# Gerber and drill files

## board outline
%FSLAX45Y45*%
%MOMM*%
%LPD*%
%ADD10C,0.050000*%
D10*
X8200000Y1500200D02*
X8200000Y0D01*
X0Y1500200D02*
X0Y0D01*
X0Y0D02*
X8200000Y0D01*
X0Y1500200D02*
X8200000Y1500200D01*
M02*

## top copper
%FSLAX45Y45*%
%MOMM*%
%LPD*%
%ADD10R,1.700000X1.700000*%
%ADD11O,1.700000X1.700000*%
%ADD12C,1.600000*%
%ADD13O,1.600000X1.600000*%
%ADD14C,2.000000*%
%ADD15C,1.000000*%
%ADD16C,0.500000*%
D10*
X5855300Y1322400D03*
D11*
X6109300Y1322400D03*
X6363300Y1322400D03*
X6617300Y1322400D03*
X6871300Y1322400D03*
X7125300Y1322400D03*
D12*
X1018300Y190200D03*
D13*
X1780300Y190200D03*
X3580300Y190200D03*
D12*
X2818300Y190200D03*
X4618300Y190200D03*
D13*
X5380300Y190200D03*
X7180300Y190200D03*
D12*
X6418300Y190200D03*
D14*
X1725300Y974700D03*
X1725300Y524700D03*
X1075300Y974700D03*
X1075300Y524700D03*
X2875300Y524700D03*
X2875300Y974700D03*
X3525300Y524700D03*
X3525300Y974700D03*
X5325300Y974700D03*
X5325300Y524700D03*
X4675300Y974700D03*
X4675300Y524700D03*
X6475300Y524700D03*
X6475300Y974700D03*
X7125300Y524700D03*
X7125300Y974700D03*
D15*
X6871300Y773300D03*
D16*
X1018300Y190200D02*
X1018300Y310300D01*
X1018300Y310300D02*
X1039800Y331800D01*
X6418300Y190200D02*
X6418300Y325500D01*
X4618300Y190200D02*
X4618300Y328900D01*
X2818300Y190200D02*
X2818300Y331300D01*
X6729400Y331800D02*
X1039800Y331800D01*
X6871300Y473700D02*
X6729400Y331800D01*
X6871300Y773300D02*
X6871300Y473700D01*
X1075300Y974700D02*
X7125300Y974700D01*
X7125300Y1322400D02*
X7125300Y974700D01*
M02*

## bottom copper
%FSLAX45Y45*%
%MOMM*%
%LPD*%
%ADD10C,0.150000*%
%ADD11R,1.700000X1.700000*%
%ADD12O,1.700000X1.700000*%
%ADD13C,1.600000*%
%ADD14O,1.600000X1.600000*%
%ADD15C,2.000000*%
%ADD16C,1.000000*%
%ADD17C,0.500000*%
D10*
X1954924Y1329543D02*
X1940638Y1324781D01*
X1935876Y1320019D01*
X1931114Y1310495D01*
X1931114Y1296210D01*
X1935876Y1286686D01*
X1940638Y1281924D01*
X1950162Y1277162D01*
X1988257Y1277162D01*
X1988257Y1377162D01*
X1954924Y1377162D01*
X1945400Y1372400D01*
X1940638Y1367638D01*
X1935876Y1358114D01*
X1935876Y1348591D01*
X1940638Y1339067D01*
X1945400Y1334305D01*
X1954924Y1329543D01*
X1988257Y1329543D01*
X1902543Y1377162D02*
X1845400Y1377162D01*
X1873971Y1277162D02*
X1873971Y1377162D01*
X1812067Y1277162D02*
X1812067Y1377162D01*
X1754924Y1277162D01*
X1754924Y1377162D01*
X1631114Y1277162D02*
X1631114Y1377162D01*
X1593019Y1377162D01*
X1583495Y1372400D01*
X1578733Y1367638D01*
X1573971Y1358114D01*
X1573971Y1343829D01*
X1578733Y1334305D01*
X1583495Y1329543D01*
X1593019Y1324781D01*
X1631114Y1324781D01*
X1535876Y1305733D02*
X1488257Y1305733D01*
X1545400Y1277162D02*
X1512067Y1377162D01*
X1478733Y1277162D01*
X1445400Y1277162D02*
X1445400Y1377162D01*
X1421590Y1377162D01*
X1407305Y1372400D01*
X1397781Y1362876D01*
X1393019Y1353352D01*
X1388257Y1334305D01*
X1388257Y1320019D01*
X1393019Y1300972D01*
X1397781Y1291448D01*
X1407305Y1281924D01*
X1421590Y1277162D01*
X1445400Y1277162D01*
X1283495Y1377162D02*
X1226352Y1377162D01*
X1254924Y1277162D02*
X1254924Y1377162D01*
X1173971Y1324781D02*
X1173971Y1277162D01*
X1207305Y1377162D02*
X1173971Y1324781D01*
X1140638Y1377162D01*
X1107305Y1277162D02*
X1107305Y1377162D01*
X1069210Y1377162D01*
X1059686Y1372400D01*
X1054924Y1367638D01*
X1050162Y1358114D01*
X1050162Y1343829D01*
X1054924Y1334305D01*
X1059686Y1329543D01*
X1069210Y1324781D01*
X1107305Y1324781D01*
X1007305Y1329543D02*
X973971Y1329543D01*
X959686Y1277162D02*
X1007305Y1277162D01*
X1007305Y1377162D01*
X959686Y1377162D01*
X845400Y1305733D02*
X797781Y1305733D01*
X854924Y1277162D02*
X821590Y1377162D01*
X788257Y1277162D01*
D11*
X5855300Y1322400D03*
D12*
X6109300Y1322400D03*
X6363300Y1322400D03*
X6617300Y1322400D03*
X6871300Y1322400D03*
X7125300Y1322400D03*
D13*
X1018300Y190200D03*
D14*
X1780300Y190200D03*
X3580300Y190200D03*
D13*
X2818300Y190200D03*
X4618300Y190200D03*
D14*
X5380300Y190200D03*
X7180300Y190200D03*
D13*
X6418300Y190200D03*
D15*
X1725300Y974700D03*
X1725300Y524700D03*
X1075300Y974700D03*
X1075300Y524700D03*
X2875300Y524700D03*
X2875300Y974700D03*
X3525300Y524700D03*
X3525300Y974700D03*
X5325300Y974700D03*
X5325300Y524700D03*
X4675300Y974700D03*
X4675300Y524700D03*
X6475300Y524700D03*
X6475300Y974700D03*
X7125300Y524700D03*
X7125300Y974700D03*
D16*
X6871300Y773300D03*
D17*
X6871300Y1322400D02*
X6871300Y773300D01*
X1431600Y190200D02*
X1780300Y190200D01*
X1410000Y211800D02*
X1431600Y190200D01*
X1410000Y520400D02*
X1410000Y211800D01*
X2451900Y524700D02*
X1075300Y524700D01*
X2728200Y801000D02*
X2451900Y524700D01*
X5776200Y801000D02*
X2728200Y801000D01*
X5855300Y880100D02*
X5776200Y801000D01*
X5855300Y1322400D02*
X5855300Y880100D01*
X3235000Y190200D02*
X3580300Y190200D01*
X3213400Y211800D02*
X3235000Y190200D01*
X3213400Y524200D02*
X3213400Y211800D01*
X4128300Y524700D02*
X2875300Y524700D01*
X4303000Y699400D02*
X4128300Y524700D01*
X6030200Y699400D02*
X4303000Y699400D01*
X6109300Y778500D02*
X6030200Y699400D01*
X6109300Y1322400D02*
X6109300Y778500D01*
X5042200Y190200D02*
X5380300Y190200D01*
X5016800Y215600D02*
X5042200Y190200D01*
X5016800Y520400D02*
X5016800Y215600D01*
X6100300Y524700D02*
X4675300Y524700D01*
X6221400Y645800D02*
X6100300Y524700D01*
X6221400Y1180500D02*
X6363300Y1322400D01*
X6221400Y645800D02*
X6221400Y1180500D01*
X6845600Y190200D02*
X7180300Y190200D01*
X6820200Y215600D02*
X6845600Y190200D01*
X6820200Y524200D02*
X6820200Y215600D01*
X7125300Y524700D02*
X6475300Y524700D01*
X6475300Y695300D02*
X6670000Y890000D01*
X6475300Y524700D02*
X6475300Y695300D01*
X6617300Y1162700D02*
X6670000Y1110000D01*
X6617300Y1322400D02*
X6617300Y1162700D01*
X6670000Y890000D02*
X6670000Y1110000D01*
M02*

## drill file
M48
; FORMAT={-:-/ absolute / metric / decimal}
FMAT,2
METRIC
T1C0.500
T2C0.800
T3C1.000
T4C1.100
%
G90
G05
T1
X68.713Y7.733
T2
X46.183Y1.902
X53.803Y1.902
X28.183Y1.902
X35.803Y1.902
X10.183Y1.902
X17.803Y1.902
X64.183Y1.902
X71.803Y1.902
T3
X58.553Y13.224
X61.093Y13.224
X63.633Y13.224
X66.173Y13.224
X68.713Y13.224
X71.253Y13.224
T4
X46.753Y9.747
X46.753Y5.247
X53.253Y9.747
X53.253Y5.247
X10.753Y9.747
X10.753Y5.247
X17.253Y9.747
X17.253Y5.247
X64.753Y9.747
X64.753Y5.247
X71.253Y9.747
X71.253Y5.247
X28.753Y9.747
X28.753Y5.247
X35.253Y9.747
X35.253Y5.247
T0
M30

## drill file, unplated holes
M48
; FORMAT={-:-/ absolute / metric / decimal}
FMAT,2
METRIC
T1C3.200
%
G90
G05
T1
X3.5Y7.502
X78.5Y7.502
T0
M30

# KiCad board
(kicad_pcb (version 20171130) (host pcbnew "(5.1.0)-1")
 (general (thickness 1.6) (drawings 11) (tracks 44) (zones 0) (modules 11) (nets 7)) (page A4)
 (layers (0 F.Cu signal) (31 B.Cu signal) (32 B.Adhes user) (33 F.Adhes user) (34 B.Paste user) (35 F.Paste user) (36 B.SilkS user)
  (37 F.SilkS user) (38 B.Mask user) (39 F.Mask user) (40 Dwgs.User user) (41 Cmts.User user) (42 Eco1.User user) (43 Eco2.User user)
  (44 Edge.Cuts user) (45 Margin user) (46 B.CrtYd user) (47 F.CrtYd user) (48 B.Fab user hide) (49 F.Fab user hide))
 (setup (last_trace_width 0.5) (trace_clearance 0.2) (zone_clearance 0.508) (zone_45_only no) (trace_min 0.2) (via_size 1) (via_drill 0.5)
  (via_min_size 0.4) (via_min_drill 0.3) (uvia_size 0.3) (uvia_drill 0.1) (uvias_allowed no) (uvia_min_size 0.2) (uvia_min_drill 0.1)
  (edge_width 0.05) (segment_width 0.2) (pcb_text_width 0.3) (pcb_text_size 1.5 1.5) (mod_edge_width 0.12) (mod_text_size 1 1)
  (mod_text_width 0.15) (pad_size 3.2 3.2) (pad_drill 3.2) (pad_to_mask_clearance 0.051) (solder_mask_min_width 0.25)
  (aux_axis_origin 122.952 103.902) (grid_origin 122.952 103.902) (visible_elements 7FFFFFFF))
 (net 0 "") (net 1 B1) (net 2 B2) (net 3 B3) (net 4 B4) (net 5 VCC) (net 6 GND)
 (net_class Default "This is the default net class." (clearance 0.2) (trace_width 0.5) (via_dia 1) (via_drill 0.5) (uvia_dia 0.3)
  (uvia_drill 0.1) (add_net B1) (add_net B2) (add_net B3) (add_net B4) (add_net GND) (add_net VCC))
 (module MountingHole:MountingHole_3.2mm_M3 (layer F.Cu) (at 201.452 96.4)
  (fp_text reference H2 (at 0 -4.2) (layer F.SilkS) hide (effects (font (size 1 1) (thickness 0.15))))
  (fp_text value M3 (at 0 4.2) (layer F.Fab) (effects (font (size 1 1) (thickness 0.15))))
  (pad 1 np_thru_hole circle (at 0 0) (size 3.2 3.2) (drill 3.2) (layers *.Cu *.Mask)))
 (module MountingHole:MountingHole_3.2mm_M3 (layer F.Cu) (at 126.452 96.4)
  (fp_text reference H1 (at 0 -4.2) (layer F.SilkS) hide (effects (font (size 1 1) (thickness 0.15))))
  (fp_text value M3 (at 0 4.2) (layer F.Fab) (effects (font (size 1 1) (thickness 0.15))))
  (pad "" np_thru_hole circle (at 0 0) (size 3.2 3.2) (drill 3.2) (layers *.Cu *.Mask)))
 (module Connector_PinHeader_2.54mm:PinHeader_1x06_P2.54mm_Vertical (layer F.Cu) (at 181.505 90.678 90)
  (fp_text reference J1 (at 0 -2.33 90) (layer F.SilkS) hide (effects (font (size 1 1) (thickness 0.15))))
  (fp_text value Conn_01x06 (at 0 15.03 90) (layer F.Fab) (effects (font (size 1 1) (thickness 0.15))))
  (pad 1 thru_hole rect (at 0 0 90) (size 1.7 1.7) (drill 1) (layers *.Cu *.Mask) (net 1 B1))
  (pad 2 thru_hole oval (at 0 2.54 90) (size 1.7 1.7) (drill 1) (layers *.Cu *.Mask) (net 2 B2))
  (pad 3 thru_hole oval (at 0 5.08 90) (size 1.7 1.7) (drill 1) (layers *.Cu *.Mask) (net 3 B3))
  (pad 4 thru_hole oval (at 0 7.62 90) (size 1.7 1.7) (drill 1) (layers *.Cu *.Mask) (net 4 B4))
  (pad 5 thru_hole oval (at 0 10.16 90) (size 1.7 1.7) (drill 1) (layers *.Cu *.Mask) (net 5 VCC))
  (pad 6 thru_hole oval (at 0 12.7 90) (size 1.7 1.7) (drill 1) (layers *.Cu *.Mask) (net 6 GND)))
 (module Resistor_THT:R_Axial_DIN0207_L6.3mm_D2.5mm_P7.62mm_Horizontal (layer F.Cu) (at 133.135 102)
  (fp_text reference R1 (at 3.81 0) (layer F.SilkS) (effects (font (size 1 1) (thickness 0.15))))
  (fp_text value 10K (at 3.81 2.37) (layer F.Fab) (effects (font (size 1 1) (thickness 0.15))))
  (pad 1 thru_hole circle (at 0 0) (size 1.6 1.6) (drill 0.8) (layers *.Cu *.Mask) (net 5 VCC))
  (pad 2 thru_hole oval (at 7.62 0) (size 1.6 1.6) (drill 0.8) (layers *.Cu *.Mask) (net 1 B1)))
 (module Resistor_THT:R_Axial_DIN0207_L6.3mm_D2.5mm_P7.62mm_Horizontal (layer F.Cu) (at 151.135 102)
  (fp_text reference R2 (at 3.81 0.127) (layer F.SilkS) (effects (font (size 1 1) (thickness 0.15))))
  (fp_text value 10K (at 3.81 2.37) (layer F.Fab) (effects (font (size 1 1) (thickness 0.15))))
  (pad 2 thru_hole oval (at 7.62 0) (size 1.6 1.6) (drill 0.8) (layers *.Cu *.Mask) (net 2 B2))
  (pad 1 thru_hole circle (at 0 0) (size 1.6 1.6) (drill 0.8) (layers *.Cu *.Mask) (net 5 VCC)))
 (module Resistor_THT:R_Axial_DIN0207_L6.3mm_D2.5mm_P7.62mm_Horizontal (layer F.Cu) (at 169.135 102)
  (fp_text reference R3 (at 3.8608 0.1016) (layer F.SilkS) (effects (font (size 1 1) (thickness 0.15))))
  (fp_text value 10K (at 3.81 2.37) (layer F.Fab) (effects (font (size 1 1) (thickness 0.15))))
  (pad 1 thru_hole circle (at 0 0) (size 1.6 1.6) (drill 0.8) (layers *.Cu *.Mask) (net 5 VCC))
  (pad 2 thru_hole oval (at 7.62 0) (size 1.6 1.6) (drill 0.8) (layers *.Cu *.Mask) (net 3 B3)))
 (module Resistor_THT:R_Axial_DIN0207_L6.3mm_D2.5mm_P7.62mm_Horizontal (layer F.Cu) (at 187.135 102)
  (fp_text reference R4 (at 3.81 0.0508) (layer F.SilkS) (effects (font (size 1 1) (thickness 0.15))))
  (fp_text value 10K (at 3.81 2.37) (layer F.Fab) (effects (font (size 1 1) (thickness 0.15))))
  (pad 2 thru_hole oval (at 7.62 0) (size 1.6 1.6) (drill 0.8) (layers *.Cu *.Mask) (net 4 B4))
  (pad 1 thru_hole circle (at 0 0) (size 1.6 1.6) (drill 0.8) (layers *.Cu *.Mask) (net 5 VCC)))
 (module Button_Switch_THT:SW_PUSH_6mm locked (layer F.Cu) (at 133.705 94.155)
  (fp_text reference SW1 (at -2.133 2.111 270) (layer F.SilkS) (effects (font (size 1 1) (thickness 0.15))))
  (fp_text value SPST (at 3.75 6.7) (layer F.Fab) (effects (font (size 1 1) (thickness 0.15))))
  (pad 1 thru_hole circle (at 6.5 0 90) (size 2 2) (drill 1.1) (layers *.Cu *.Mask) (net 6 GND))
  (pad 2 thru_hole circle (at 6.5 4.5 90) (size 2 2) (drill 1.1) (layers *.Cu *.Mask) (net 1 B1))
  (pad 1 thru_hole circle (at 0 0 90) (size 2 2) (drill 1.1) (layers *.Cu *.Mask) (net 6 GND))
  (pad 2 thru_hole circle (at 0 4.5 90) (size 2 2) (drill 1.1) (layers *.Cu *.Mask) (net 1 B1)))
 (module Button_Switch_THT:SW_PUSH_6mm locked (layer F.Cu) (at 151.705 94.155)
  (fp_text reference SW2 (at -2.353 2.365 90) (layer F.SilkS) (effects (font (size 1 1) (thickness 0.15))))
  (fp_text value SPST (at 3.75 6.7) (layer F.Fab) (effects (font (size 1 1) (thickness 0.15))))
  (pad 2 thru_hole circle (at 0 4.5 90) (size 2 2) (drill 1.1) (layers *.Cu *.Mask) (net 2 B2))
  (pad 1 thru_hole circle (at 0 0 90) (size 2 2) (drill 1.1) (layers *.Cu *.Mask) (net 6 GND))
  (pad 2 thru_hole circle (at 6.5 4.5 90) (size 2 2) (drill 1.1) (layers *.Cu *.Mask) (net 2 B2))
  (pad 1 thru_hole circle (at 6.5 0 90) (size 2 2) (drill 1.1) (layers *.Cu *.Mask) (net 6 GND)))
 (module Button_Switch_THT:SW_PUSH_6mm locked (layer F.Cu) (at 169.705 94.155)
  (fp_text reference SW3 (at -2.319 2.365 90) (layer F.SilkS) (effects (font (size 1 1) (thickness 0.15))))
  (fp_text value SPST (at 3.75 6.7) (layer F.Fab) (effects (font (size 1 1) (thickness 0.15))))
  (pad 1 thru_hole circle (at 6.5 0 90) (size 2 2) (drill 1.1) (layers *.Cu *.Mask) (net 6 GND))
  (pad 2 thru_hole circle (at 6.5 4.5 90) (size 2 2) (drill 1.1) (layers *.Cu *.Mask) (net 3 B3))
  (pad 1 thru_hole circle (at 0 0 90) (size 2 2) (drill 1.1) (layers *.Cu *.Mask) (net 6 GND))
  (pad 2 thru_hole circle (at 0 4.5 90) (size 2 2) (drill 1.1) (layers *.Cu *.Mask) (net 3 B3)))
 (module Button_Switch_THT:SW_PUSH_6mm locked (layer F.Cu) (at 187.705 94.155)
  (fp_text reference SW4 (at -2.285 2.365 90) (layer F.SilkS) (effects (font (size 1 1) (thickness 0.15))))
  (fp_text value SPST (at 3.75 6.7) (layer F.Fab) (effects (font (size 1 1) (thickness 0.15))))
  (pad 2 thru_hole circle (at 0 4.5 90) (size 2 2) (drill 1.1) (layers *.Cu *.Mask) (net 4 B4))
  (pad 1 thru_hole circle (at 0 0 90) (size 2 2) (drill 1.1) (layers *.Cu *.Mask) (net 6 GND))
  (pad 2 thru_hole circle (at 6.5 4.5 90) (size 2 2) (drill 1.1) (layers *.Cu *.Mask) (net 4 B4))
  (pad 1 thru_hole circle (at 6.5 0 90) (size 2 2) (drill 1.1) (layers *.Cu *.Mask) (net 6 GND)))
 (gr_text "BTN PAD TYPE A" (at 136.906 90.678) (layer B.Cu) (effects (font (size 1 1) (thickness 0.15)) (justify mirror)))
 (gr_line (start 204.952 88.9) (end 204.952 103.902) (layer Edge.Cuts) (width 0.05))
 (gr_line (start 122.952 88.9) (end 122.952 103.902) (layer Edge.Cuts) (width 0.05))
 (gr_line (start 122.952 103.902) (end 204.952 103.902) (layer Edge.Cuts) (width 0.05))
 (gr_line (start 122.952 88.9) (end 204.952 88.9) (layer Edge.Cuts) (width 0.05))
 (segment (start 133.135 102) (end 133.135 100.799) (width 0.5) (layer F.Cu) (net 5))
 (segment (start 133.135 100.799) (end 133.35 100.584) (width 0.5) (layer F.Cu) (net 5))
 (segment (start 187.135 102) (end 187.135 100.647) (width 0.5) (layer F.Cu) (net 5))
 (segment (start 169.135 102) (end 169.135 100.613) (width 0.5) (layer F.Cu) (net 5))
 (segment (start 151.135 102) (end 151.135 100.589) (width 0.5) (layer F.Cu) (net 5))
 (segment (start 190.246 100.584) (end 133.35 100.584) (width 0.5) (layer F.Cu) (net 5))
 (via (at 191.665 96.169) (size 1) (drill 0.5) (layers F.Cu B.Cu) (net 5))
 (segment (start 191.665 90.678) (end 191.665 96.169) (width 0.5) (layer B.Cu) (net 5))
 (segment (start 191.665 99.165) (end 190.246 100.584) (width 0.5) (layer F.Cu) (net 5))
 (segment (start 191.665 96.169) (end 191.665 99.165) (width 0.5) (layer F.Cu) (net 5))
 (segment (start 133.705 94.155) (end 194.205 94.155) (width 0.5) (layer F.Cu) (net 6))
 (segment (start 194.205 90.678) (end 194.205 94.155) (width 0.5) (layer F.Cu) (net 6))
 (segment (start 137.268 102) (end 140.755 102) (width 0.5) (layer B.Cu) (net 1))
 (segment (start 137.052 101.784) (end 137.268 102) (width 0.5) (layer B.Cu) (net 1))
 (segment (start 137.052 98.698) (end 137.052 101.784) (width 0.5) (layer B.Cu) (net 1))
 (segment (start 147.471 98.655) (end 133.705 98.655) (width 0.5) (layer B.Cu) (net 1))
 (segment (start 150.234 95.892) (end 147.471 98.655) (width 0.5) (layer B.Cu) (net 1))
 (segment (start 180.714 95.892) (end 150.234 95.892) (width 0.5) (layer B.Cu) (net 1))
 (segment (start 181.505 95.101) (end 180.714 95.892) (width 0.5) (layer B.Cu) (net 1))
 (segment (start 181.505 90.678) (end 181.505 95.101) (width 0.5) (layer B.Cu) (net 1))
 (segment (start 155.302 102) (end 158.755 102) (width 0.5) (layer B.Cu) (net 2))
 (segment (start 155.086 101.784) (end 155.302 102) (width 0.5) (layer B.Cu) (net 2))
 (segment (start 155.086 98.66) (end 155.086 101.784) (width 0.5) (layer B.Cu) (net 2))
 (segment (start 164.235 98.655) (end 151.705 98.655) (width 0.5) (layer B.Cu) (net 2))
 (segment (start 165.982 96.908) (end 164.235 98.655) (width 0.5) (layer B.Cu) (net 2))
 (segment (start 183.254 96.908) (end 165.982 96.908) (width 0.5) (layer B.Cu) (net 2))
 (segment (start 184.045 96.117) (end 183.254 96.908) (width 0.5) (layer B.Cu) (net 2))
 (segment (start 184.045 90.678) (end 184.045 96.117) (width 0.5) (layer B.Cu) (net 2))
 (segment (start 173.374 102) (end 176.755 102) (width 0.5) (layer B.Cu) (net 3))
 (segment (start 173.12 101.746) (end 173.374 102) (width 0.5) (layer B.Cu) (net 3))
 (segment (start 173.12 98.698) (end 173.12 101.746) (width 0.5) (layer B.Cu) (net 3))
 (segment (start 183.955 98.655) (end 169.705 98.655) (width 0.5) (layer B.Cu) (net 3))
 (segment (start 185.166 97.444) (end 183.955 98.655) (width 0.5) (layer B.Cu) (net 3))
 (segment (start 185.166 92.097) (end 186.585 90.678) (width 0.5) (layer B.Cu) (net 3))
 (segment (start 185.166 97.444) (end 185.166 92.097) (width 0.5) (layer B.Cu) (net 3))
 (segment (start 191.408 102) (end 194.755 102) (width 0.5) (layer B.Cu) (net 4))
 (segment (start 191.154 101.746) (end 191.408 102) (width 0.5) (layer B.Cu) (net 4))
 (segment (start 191.154 98.66) (end 191.154 101.746) (width 0.5) (layer B.Cu) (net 4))
 (segment (start 194.205 98.655) (end 187.705 98.655) (width 0.5) (layer B.Cu) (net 4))
 (segment (start 187.705 96.949) (end 189.652 95.002) (width 0.5) (layer B.Cu) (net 4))
 (segment (start 187.705 98.655) (end 187.705 96.949) (width 0.5) (layer B.Cu) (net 4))
 (segment (start 189.125 92.275) (end 189.652 92.802) (width 0.5) (layer B.Cu) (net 4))
 (segment (start 189.125 90.678) (end 189.125 92.275) (width 0.5) (layer B.Cu) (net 4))
 (segment (start 189.652 95.002) (end 189.652 92.802) (width 0.5) (layer B.Cu) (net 4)))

